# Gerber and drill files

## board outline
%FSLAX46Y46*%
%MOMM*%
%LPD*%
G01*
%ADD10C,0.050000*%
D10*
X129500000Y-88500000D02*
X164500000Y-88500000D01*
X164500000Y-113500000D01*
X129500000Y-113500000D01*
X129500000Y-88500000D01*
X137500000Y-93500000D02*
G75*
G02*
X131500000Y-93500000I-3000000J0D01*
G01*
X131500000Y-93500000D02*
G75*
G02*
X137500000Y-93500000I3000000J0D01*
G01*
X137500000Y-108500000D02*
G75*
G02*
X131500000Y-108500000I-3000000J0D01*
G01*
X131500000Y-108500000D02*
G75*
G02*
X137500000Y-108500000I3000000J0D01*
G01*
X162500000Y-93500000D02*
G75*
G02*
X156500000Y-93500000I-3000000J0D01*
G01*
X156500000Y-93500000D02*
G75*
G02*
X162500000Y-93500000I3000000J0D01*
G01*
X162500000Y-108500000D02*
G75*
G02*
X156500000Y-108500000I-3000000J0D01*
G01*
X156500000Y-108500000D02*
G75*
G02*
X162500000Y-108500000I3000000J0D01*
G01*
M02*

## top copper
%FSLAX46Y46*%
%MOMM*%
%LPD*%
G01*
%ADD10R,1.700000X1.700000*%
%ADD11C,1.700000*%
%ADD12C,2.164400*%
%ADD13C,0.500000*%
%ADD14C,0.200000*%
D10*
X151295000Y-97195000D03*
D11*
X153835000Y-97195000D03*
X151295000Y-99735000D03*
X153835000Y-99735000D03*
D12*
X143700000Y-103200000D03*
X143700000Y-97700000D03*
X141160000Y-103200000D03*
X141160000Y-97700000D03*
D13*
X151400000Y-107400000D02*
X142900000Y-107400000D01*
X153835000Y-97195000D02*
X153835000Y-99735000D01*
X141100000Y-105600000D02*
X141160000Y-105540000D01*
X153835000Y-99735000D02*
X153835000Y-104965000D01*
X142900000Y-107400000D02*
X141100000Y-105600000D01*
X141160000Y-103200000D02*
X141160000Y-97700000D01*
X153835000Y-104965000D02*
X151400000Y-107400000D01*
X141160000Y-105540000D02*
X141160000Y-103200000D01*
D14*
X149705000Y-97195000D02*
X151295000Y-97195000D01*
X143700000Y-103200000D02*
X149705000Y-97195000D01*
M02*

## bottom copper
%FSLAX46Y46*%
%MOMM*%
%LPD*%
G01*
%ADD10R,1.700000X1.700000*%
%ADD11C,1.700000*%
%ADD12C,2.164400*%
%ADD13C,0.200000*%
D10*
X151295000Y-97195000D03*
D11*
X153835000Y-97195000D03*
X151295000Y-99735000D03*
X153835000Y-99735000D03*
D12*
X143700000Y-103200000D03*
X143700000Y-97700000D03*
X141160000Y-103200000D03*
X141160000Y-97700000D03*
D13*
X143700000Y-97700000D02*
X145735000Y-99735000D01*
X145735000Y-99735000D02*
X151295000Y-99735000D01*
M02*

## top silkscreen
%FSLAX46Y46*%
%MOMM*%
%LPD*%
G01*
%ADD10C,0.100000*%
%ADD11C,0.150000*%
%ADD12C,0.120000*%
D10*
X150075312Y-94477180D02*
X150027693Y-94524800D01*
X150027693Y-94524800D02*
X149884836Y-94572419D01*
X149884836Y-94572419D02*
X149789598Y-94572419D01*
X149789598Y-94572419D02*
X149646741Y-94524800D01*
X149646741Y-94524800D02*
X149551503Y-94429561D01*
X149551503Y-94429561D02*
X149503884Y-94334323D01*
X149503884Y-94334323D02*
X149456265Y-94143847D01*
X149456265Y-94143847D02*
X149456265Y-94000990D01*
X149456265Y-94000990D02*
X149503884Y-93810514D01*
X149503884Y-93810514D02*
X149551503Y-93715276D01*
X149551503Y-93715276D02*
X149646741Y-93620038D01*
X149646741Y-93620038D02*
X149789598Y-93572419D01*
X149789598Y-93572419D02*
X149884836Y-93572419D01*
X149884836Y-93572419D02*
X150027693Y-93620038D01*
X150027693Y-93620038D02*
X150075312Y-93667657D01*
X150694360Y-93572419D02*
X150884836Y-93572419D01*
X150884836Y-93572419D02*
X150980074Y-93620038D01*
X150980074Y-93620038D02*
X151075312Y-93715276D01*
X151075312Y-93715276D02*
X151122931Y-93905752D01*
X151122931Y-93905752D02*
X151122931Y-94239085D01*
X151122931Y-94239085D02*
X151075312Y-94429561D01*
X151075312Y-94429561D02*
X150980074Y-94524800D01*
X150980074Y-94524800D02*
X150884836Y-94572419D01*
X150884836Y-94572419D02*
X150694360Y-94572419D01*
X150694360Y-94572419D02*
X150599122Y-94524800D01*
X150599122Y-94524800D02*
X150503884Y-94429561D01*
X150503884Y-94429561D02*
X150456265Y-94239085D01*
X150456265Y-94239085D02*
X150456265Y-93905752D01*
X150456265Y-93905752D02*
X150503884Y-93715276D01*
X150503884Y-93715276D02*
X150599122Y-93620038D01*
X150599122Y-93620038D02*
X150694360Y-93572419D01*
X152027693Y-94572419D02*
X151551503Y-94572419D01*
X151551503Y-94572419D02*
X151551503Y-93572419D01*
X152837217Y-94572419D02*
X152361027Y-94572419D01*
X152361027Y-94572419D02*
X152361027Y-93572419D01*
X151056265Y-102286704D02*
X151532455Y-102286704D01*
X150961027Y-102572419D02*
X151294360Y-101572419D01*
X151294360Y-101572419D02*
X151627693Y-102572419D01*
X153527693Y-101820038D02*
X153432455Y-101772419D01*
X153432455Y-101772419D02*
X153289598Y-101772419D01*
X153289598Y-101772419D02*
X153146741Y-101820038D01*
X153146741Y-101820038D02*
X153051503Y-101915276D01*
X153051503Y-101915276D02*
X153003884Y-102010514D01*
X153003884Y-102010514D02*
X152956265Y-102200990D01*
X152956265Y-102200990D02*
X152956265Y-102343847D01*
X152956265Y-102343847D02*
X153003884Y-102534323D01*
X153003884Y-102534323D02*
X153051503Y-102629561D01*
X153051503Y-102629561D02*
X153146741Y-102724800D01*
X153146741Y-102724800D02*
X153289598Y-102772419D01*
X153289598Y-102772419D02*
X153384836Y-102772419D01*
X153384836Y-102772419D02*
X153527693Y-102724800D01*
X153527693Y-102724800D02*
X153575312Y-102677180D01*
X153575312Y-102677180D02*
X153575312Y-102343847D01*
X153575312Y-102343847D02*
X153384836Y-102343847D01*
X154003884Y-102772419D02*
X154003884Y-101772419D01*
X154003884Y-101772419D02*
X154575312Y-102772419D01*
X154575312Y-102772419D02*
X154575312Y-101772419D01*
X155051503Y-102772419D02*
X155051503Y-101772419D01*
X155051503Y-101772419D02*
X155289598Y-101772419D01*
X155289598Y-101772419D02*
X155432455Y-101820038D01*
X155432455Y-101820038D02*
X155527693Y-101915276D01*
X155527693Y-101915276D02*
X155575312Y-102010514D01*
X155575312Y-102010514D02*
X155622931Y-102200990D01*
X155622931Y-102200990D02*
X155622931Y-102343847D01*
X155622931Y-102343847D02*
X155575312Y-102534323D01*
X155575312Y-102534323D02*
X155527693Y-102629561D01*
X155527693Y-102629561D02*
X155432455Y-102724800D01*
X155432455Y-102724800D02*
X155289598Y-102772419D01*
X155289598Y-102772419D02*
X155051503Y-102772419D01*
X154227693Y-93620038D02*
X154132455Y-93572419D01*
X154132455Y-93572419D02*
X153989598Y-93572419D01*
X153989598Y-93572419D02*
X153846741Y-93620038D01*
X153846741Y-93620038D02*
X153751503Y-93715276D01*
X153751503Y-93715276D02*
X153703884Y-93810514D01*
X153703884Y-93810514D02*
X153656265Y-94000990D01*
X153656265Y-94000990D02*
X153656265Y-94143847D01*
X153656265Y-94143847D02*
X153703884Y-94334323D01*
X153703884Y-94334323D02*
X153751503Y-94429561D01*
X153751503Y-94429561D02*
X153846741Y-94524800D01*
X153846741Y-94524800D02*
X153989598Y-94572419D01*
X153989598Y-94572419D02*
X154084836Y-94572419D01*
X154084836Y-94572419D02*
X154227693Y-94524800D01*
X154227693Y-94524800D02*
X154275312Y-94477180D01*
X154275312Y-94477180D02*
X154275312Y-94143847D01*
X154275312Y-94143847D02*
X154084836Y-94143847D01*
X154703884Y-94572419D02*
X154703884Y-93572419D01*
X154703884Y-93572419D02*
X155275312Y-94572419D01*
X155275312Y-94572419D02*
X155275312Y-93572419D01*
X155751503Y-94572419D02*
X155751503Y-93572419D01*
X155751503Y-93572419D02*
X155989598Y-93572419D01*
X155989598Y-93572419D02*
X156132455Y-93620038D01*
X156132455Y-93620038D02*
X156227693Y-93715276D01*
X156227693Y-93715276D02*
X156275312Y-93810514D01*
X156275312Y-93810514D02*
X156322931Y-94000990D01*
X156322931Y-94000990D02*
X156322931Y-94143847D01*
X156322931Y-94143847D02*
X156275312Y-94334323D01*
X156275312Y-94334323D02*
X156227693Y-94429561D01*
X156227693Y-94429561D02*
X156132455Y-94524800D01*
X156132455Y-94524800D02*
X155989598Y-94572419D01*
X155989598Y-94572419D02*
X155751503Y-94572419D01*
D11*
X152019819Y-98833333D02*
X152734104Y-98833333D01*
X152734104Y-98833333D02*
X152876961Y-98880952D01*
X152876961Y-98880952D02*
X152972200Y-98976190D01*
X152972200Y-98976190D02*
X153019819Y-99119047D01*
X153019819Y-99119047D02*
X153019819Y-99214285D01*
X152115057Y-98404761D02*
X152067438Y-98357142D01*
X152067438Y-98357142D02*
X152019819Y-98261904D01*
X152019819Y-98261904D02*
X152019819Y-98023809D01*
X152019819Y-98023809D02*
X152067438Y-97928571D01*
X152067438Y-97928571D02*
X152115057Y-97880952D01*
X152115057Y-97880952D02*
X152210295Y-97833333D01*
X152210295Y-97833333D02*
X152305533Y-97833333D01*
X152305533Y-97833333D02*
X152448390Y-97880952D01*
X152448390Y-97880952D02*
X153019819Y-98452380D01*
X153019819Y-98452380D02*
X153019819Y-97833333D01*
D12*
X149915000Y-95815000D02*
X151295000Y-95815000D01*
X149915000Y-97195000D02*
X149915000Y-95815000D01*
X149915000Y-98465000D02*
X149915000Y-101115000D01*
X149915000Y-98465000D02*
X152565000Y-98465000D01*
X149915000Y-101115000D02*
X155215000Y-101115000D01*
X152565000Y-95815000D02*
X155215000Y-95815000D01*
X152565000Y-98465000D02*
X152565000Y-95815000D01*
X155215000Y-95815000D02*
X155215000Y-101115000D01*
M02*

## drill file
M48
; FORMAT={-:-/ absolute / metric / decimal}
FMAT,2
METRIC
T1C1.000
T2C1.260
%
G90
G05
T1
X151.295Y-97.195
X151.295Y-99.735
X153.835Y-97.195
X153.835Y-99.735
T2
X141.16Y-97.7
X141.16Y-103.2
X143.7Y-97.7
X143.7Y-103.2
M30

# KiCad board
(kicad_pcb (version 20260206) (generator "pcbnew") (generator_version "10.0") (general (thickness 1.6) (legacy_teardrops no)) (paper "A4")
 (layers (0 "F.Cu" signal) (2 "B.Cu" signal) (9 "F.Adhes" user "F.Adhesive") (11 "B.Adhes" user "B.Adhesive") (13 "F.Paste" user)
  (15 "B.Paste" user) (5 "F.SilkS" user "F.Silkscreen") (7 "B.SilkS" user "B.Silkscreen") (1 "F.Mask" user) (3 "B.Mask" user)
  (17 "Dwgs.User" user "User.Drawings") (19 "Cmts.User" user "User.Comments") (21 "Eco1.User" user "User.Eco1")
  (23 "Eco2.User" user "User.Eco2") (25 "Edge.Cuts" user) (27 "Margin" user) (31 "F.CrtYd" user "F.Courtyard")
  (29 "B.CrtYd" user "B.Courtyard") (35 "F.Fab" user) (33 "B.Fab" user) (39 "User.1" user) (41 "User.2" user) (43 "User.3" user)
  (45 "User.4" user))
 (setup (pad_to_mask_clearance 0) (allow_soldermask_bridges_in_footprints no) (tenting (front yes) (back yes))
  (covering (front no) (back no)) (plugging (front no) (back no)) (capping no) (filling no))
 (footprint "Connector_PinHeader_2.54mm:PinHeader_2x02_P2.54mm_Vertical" (layer "F.Cu") (at 151.295 97.195)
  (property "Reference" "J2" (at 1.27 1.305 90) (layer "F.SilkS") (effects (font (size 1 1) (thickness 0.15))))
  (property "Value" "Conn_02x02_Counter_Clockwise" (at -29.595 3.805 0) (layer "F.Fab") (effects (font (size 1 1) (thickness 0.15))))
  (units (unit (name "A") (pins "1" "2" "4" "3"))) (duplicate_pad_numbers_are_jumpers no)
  (fp_line (start -1.38 -1.38) (end 0 -1.38) (stroke (width 0.12) (type solid)) (layer "F.SilkS"))
  (fp_line (start -1.38 0) (end -1.38 -1.38) (stroke (width 0.12) (type solid)) (layer "F.SilkS"))
  (fp_line (start -1.38 1.27) (end -1.38 3.92) (stroke (width 0.12) (type solid)) (layer "F.SilkS"))
  (fp_line (start -1.38 1.27) (end 1.27 1.27) (stroke (width 0.12) (type solid)) (layer "F.SilkS"))
  (fp_line (start -1.38 3.92) (end 3.92 3.92) (stroke (width 0.12) (type solid)) (layer "F.SilkS"))
  (fp_line (start 1.27 -1.38) (end 3.92 -1.38) (stroke (width 0.12) (type solid)) (layer "F.SilkS"))
  (fp_line (start 1.27 1.27) (end 1.27 -1.38) (stroke (width 0.12) (type solid)) (layer "F.SilkS"))
  (fp_line (start 3.92 -1.38) (end 3.92 3.92) (stroke (width 0.12) (type solid)) (layer "F.SilkS"))
  (pad "1" thru_hole rect (at 0 0) (size 1.7 1.7) (drill 1) (layers "*.Cu" "*.Mask") (remove_unused_layers no) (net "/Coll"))
  (pad "2" thru_hole circle (at 2.54 0) (size 1.7 1.7) (drill 1) (layers "*.Cu" "*.Mask") (remove_unused_layers no) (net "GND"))
  (pad "3" thru_hole circle (at 0 2.54) (size 1.7 1.7) (drill 1) (layers "*.Cu" "*.Mask") (remove_unused_layers no) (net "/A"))
  (pad "4" thru_hole circle (at 2.54 2.54) (size 1.7 1.7) (drill 1) (layers "*.Cu" "*.Mask") (remove_unused_layers no) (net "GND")))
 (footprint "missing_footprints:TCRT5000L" (layer "B.Cu") (at 142.43 100.45 90)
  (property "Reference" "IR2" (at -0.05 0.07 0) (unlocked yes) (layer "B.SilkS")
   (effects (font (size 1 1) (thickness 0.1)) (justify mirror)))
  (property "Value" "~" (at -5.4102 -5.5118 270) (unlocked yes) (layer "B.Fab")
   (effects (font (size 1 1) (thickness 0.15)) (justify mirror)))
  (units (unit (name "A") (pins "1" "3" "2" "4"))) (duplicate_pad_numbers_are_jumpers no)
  (pad "1" thru_hole circle (at -2.75 1.27 90) (size 2.1644 2.1644) (drill 1.26) (layers "*.Cu" "*.Mask") (remove_unused_layers no)
   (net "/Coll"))
  (pad "2" thru_hole circle (at 2.75 1.27 90) (size 2.1644 2.1644) (drill 1.26) (layers "*.Cu" "*.Mask") (remove_unused_layers no)
   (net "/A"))
  (pad "3" thru_hole circle (at -2.75 -1.27 90) (size 2.1644 2.1644) (drill 1.26) (layers "*.Cu" "*.Mask") (remove_unused_layers no)
   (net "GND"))
  (pad "4" thru_hole circle (at 2.75 -1.27 90) (size 2.1644 2.1644) (drill 1.26) (layers "*.Cu" "*.Mask") (remove_unused_layers no)
   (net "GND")))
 (gr_rect (start 129.5 88.5) (end 164.5 113.5) (stroke (width 0.05) (type solid)) (fill no) (layer "Edge.Cuts"))
 (gr_circle (center 134.5 93.5) (end 137.5 93.5) (stroke (width 0.05) (type solid)) (fill no) (layer "Edge.Cuts"))
 (gr_circle (center 134.5 108.5) (end 137.5 108.5) (stroke (width 0.05) (type solid)) (fill no) (layer "Edge.Cuts"))
 (gr_circle (center 159.5 93.5) (end 162.5 93.5) (stroke (width 0.05) (type solid)) (fill no) (layer "Edge.Cuts"))
 (gr_circle (center 159.5 108.5) (end 162.5 108.5) (stroke (width 0.05) (type solid)) (fill no) (layer "Edge.Cuts"))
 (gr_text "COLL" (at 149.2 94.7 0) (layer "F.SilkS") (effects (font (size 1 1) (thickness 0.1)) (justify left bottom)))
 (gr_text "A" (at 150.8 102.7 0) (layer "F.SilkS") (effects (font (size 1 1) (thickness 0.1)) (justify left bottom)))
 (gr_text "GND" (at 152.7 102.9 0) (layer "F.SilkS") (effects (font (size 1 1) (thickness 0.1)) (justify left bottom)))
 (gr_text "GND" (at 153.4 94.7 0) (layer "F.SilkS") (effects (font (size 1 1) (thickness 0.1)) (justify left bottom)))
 (segment (start 143.7 97.7) (end 145.735 99.735) (width 0.2) (layer "B.Cu") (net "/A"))
 (segment (start 145.735 99.735) (end 151.295 99.735) (width 0.2) (layer "B.Cu") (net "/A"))
 (segment (start 151.4 107.4) (end 142.9 107.4) (width 0.5) (layer "F.Cu") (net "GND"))
 (segment (start 153.835 97.195) (end 153.835 99.735) (width 0.5) (layer "F.Cu") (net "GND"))
 (segment (start 141.1 105.6) (end 141.16 105.54) (width 0.5) (layer "F.Cu") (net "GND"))
 (segment (start 153.835 99.735) (end 153.835 104.965) (width 0.5) (layer "F.Cu") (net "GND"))
 (segment (start 142.9 107.4) (end 141.1 105.6) (width 0.5) (layer "F.Cu") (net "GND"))
 (segment (start 141.16 103.2) (end 141.16 97.7) (width 0.5) (layer "F.Cu") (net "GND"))
 (segment (start 153.835 104.965) (end 151.4 107.4) (width 0.5) (layer "F.Cu") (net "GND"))
 (segment (start 141.16 105.54) (end 141.16 103.2) (width 0.5) (layer "F.Cu") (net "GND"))
 (segment (start 149.705 97.195) (end 151.295 97.195) (width 0.2) (layer "F.Cu") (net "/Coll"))
 (segment (start 143.7 103.2) (end 149.705 97.195) (width 0.2) (layer "F.Cu") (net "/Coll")))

